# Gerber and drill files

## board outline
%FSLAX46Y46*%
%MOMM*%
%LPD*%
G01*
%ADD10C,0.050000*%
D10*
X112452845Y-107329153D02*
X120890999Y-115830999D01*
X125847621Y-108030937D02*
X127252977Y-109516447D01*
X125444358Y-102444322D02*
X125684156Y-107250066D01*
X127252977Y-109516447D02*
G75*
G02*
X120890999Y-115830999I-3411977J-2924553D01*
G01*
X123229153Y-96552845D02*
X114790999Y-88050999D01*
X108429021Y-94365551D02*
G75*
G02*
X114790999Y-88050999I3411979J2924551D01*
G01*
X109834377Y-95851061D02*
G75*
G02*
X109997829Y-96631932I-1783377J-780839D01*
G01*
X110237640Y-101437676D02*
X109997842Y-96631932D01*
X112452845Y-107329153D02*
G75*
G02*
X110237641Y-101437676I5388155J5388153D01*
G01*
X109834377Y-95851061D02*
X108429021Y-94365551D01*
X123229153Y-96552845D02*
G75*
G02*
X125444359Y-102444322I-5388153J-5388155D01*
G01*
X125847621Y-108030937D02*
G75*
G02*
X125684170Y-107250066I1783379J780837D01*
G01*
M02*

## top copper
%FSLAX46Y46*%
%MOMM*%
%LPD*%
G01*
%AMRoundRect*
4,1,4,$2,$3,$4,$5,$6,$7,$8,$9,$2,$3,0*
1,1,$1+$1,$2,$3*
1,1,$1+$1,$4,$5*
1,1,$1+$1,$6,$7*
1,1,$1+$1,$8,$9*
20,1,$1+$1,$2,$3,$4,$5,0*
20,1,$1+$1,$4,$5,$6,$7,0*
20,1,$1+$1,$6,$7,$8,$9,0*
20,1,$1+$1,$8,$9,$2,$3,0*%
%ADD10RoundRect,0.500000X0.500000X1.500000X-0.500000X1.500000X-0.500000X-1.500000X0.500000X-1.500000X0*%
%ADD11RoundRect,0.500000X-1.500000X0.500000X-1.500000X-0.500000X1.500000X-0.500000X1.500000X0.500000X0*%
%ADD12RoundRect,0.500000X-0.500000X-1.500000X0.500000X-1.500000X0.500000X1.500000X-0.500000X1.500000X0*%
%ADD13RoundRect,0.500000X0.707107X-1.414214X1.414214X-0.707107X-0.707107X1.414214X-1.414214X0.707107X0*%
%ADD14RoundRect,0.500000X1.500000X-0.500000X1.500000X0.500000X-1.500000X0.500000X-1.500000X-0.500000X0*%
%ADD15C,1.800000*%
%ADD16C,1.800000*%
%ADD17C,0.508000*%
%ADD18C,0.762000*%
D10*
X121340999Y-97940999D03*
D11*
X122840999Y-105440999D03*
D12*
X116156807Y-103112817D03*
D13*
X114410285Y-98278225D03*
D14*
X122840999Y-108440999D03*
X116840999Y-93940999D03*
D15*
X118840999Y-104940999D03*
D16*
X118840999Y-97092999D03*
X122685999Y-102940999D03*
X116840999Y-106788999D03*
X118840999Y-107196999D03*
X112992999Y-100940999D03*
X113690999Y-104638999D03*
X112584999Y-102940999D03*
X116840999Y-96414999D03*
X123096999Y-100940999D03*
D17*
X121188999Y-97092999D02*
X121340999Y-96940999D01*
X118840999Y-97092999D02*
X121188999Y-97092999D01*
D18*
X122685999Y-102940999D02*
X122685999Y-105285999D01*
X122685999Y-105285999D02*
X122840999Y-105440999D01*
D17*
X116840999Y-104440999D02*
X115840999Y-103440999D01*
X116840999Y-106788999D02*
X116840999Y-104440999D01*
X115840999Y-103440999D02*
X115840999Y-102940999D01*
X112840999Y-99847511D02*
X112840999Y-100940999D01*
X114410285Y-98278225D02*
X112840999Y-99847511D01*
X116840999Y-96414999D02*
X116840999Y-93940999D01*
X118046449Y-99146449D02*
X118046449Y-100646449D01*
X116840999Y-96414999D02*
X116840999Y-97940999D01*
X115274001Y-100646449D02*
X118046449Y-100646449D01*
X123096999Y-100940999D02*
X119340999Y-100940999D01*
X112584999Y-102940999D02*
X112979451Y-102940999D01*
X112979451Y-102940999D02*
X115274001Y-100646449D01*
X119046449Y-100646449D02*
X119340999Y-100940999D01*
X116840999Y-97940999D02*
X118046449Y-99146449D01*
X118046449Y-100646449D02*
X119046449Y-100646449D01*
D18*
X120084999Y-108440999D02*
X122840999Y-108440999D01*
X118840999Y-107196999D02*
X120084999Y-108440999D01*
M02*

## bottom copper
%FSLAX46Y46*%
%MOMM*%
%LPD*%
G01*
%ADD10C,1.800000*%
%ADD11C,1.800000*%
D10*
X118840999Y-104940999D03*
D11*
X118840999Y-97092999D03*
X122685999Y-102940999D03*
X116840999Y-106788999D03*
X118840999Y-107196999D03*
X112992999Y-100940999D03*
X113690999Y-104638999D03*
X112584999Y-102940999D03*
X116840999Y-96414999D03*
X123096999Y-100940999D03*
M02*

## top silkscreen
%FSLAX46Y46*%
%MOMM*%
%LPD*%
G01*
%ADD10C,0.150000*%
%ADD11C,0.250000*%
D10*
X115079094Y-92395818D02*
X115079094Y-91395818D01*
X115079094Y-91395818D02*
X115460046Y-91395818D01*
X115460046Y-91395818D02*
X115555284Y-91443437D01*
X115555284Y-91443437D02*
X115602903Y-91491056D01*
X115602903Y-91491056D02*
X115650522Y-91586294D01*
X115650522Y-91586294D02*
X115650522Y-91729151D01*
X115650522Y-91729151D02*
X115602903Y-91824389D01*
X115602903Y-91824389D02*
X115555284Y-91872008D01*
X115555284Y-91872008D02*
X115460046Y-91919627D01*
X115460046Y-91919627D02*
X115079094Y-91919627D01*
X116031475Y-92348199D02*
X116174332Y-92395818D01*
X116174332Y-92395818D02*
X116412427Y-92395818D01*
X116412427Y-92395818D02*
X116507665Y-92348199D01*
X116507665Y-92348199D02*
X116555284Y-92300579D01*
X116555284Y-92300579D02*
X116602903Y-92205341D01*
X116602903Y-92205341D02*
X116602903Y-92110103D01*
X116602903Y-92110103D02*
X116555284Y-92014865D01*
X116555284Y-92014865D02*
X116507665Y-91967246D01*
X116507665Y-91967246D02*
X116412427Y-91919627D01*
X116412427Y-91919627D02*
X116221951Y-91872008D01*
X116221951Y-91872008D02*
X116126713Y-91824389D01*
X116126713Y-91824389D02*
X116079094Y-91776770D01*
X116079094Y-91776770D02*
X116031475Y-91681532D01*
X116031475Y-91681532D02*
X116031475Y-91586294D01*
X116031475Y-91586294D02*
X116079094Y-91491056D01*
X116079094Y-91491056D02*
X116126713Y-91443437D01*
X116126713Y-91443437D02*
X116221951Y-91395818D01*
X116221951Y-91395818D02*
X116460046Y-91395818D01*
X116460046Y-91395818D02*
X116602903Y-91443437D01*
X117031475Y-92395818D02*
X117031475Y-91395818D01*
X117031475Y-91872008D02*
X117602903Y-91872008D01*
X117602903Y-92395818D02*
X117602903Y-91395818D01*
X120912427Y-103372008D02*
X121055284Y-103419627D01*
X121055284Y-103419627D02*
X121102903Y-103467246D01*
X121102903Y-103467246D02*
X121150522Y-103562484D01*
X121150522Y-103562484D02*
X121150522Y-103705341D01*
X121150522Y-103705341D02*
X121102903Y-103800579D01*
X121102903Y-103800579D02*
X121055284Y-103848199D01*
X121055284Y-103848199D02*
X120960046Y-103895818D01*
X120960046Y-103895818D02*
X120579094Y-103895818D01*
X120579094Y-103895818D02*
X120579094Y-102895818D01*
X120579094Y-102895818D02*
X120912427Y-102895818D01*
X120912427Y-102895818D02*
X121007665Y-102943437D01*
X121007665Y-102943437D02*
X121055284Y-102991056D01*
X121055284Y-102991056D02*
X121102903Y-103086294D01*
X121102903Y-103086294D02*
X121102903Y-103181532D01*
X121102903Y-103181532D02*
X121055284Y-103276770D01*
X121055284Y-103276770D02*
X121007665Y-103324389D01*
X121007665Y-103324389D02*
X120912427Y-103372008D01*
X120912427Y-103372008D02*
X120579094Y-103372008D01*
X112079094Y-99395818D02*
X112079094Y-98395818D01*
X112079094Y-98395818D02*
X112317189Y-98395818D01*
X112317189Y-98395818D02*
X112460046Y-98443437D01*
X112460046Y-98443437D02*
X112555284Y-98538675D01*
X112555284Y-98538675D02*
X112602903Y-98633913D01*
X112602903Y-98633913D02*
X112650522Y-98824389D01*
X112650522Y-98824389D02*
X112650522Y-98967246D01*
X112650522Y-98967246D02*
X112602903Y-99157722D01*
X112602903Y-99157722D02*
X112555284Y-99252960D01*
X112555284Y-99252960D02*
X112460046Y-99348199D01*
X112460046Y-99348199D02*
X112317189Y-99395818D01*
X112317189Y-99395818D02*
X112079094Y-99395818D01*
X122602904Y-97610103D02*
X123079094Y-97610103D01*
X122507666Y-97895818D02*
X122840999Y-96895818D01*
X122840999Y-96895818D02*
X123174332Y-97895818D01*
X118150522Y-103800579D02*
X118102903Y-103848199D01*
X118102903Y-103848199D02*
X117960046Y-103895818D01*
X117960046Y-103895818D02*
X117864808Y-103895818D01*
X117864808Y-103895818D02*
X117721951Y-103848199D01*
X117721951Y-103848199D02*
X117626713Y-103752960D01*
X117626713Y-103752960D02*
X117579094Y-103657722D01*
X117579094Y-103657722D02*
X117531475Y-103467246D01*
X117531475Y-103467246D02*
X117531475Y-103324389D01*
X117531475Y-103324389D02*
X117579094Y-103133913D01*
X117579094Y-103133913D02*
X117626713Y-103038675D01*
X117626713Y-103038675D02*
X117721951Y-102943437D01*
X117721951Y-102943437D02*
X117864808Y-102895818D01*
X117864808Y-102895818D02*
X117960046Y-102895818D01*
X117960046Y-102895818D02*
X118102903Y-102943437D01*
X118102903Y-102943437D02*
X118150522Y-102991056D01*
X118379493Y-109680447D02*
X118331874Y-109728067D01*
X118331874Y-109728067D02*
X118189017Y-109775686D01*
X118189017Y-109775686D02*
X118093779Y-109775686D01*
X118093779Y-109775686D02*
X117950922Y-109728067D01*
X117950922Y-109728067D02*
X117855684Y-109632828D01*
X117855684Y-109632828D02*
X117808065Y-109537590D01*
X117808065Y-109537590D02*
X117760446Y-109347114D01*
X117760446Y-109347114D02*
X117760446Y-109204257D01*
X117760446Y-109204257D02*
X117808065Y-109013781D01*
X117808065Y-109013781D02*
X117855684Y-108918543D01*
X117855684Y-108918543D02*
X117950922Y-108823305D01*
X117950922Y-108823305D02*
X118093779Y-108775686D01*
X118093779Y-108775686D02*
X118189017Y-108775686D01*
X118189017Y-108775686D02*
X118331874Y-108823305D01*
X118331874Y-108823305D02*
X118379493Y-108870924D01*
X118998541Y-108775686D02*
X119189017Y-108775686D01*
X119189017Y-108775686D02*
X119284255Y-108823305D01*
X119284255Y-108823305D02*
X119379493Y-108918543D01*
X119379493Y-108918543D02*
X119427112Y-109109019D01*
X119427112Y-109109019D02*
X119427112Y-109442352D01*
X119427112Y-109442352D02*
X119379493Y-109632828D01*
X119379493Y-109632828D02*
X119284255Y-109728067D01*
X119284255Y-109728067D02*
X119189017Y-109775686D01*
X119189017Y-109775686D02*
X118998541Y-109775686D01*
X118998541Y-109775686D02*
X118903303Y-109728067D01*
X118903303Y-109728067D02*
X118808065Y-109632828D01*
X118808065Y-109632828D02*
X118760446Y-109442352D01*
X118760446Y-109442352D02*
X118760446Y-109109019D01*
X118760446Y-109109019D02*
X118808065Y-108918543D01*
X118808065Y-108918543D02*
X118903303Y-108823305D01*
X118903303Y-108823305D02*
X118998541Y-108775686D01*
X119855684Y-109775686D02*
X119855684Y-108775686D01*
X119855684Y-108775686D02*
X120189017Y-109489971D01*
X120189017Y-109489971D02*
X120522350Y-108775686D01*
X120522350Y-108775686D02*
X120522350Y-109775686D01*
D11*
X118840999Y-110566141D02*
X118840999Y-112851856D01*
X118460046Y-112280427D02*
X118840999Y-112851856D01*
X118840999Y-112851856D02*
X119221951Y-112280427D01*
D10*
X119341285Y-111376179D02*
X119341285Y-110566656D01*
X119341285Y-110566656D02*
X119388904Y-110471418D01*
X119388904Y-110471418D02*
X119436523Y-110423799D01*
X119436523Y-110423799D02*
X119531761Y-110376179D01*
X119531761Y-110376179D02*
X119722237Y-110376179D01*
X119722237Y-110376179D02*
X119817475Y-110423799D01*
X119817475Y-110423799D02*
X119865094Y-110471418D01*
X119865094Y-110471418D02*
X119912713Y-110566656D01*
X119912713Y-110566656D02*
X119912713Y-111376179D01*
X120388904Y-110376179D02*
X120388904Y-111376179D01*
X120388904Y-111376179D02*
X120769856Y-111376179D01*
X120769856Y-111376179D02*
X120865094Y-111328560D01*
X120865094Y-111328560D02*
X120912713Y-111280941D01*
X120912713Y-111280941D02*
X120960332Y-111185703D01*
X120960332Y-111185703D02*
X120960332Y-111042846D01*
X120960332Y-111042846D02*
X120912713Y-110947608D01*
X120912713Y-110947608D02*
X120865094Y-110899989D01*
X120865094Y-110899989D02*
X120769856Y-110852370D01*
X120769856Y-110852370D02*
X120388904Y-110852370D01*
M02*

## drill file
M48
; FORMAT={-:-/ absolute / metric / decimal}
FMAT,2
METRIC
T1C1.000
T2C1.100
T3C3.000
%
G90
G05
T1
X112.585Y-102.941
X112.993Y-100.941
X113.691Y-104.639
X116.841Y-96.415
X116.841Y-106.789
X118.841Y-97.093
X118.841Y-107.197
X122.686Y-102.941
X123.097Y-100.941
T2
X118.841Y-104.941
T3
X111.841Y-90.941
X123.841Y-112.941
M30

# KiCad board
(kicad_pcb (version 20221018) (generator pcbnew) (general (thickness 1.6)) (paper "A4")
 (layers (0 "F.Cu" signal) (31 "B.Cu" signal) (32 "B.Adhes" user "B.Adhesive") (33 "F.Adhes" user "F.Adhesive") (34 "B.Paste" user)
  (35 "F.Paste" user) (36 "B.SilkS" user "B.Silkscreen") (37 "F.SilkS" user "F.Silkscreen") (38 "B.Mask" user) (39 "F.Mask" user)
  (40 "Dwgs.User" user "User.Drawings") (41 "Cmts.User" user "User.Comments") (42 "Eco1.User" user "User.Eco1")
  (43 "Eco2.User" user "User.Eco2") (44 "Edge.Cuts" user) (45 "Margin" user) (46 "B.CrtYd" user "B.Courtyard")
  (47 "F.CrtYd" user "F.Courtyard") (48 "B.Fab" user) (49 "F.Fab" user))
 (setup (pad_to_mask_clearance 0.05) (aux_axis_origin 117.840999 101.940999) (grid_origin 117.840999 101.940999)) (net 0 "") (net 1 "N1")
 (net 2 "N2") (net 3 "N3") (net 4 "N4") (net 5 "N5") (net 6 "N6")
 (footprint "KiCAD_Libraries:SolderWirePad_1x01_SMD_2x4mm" (layer "F.Cu") (at 121.340999 97.940999 180)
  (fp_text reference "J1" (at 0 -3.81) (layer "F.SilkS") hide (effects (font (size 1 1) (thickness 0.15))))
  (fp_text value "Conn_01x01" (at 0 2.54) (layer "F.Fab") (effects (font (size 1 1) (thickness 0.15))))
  (pad "1" smd roundrect (at 0 0 180) (size 2 4) (layers "F.Cu" "F.Paste" "F.Mask") (roundrect_rratio 0.25) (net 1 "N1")))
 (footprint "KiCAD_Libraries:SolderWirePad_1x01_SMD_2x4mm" (layer "F.Cu") (at 122.840999 105.440999 -90)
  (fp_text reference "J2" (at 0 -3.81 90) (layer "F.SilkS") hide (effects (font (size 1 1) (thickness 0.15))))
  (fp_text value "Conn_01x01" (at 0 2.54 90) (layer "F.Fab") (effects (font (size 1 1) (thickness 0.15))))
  (pad "1" smd roundrect (at 0 0 270) (size 2 4) (layers "F.Cu" "F.Paste" "F.Mask") (roundrect_rratio 0.25) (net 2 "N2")))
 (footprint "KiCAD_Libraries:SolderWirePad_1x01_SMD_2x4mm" (layer "F.Cu") (at 116.156807 103.112817)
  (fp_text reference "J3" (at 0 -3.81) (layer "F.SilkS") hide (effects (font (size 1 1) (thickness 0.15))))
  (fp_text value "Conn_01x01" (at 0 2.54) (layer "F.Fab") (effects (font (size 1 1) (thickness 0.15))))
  (pad "1" smd roundrect (at 0 0) (size 2 4) (layers "F.Cu" "F.Paste" "F.Mask") (roundrect_rratio 0.25) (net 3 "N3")))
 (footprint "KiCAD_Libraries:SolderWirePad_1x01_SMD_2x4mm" (layer "F.Cu") (at 114.410285 98.278225 45)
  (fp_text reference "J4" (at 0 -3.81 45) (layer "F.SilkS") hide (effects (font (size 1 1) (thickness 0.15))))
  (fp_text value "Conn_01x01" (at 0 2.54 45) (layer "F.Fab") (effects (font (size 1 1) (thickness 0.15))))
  (pad "1" smd roundrect (at 0 0 45) (size 2 4) (layers "F.Cu" "F.Paste" "F.Mask") (roundrect_rratio 0.25) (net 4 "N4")))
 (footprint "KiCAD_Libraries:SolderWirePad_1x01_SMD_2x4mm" (layer "F.Cu") (at 122.840999 108.440999 90)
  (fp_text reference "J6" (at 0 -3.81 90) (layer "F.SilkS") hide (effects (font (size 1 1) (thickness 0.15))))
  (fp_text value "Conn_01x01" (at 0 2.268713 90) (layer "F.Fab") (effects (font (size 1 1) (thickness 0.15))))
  (pad "1" smd roundrect (at 0 0 90) (size 2 4) (layers "F.Cu" "F.Paste" "F.Mask") (roundrect_rratio 0.25) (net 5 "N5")))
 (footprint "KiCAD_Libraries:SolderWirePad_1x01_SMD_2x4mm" (layer "F.Cu") (at 116.840999 93.940999 90)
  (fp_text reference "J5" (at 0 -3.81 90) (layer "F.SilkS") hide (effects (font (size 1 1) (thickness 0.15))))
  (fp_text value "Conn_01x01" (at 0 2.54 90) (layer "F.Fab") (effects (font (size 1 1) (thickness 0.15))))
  (pad "1" smd roundrect (at 0 0 90) (size 2 4) (layers "F.Cu" "F.Paste" "F.Mask") (roundrect_rratio 0.25) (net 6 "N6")))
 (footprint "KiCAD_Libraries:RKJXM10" (layer "B.Cu") (at 117.840999 101.940999)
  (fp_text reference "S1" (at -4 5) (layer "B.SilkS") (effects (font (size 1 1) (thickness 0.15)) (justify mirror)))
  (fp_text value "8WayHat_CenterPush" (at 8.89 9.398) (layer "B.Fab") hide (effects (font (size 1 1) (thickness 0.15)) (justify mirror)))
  (pad "" np_thru_hole circle (at 1 3) (size 1.8 1.8) (drill 1.1) (layers "*.Cu" "*.Mask"))
  (pad "A" thru_hole circle (at 1 -4.848) (size 1.8 1.8) (drill 1) (layers "*.Cu" "*.Mask") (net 1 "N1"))
  (pad "B" thru_hole circle (at 4.845 1) (size 1.8 1.8) (drill 1) (layers "*.Cu" "*.Mask") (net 2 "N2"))
  (pad "C" thru_hole circle (at -1 4.848) (size 1.8 1.8) (drill 1) (layers "*.Cu" "*.Mask") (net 3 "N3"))
  (pad "COM" thru_hole circle (at 1 5.256) (size 1.8 1.8) (drill 1) (layers "*.Cu" "*.Mask") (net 5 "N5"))
  (pad "D" thru_hole circle (at -4.848 -1) (size 1.8 1.8) (drill 1) (layers "*.Cu" "*.Mask") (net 4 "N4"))
  (pad "GND" thru_hole circle (at -4.15 2.698) (size 1.8 1.8) (drill 1) (layers "*.Cu" "*.Mask"))
  (pad "PUSH1" thru_hole circle (at -5.256 1) (size 1.8 1.8) (drill 1) (layers "*.Cu" "*.Mask") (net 6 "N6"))
  (pad "PUSH2" thru_hole circle (at -1 -5.526) (size 1.8 1.8) (drill 1) (layers "*.Cu" "*.Mask") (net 6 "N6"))
  (pad "PUSH3" thru_hole circle (at 5.256 -1) (size 1.8 1.8) (drill 1) (layers "*.Cu" "*.Mask") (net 6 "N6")))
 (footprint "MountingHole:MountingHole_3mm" (layer "B.Cu") (at 123.840999 112.940999)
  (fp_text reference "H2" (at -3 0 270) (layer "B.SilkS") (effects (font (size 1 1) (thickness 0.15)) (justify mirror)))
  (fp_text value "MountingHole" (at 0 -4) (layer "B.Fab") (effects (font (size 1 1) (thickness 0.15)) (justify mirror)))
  (pad "" np_thru_hole circle (at 0 0) (size 3 3) (drill 3) (layers "*.Cu" "*.Mask")))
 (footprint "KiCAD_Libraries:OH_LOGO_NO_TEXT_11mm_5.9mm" (layer "B.Cu") (at 118.340999 101.440999 -160)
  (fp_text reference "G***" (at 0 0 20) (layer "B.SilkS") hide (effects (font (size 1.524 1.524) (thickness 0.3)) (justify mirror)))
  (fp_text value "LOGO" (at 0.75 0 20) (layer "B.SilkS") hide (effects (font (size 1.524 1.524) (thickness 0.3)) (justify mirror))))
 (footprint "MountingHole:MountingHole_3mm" (layer "B.Cu") (at 111.840999 90.940999 180)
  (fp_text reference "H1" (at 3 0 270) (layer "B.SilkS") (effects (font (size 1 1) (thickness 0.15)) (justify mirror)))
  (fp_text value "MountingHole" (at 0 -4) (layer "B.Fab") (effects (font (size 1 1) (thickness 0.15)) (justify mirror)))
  (pad "" np_thru_hole circle (at 0 0 180) (size 3 3) (drill 3) (layers "*.Cu" "*.Mask")))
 (gr_line (start 112.452845 107.329153) (end 120.890999 115.830999) (stroke (width 0.05) (type solid)) (layer "Edge.Cuts"))
 (gr_line (start 125.847621 108.030937) (end 127.252977 109.516447) (stroke (width 0.05) (type solid)) (layer "Edge.Cuts"))
 (gr_line (start 125.444358 102.444322) (end 125.684156 107.250066) (stroke (width 0.05) (type solid)) (layer "Edge.Cuts"))
 (gr_arc (start 127.252977 109.516447) (mid 127.006713 115.63049) (end 120.890999 115.830999) (stroke (width 0.05) (type solid))
  (layer "Edge.Cuts"))
 (gr_line (start 123.229153 96.552845) (end 114.790999 88.050999) (stroke (width 0.05) (type solid)) (layer "Edge.Cuts"))
 (gr_arc (start 108.429021 94.365551) (mid 108.675285 88.251508) (end 114.790999 88.050999) (stroke (width 0.05) (type solid))
  (layer "Edge.Cuts"))
 (gr_arc (start 109.834377 95.851061) (mid 109.956537 96.233033) (end 109.997842 96.631932) (stroke (width 0.05) (type solid))
  (layer "Edge.Cuts"))
 (gr_line (start 110.23764 101.437676) (end 109.997842 96.631932) (stroke (width 0.05) (type solid)) (layer "Edge.Cuts"))
 (gr_arc (start 112.452845 107.329153) (mid 110.708522 104.622822) (end 110.23764 101.437676) (stroke (width 0.05) (type solid))
  (layer "Edge.Cuts"))
 (gr_line (start 109.834377 95.851061) (end 108.429021 94.365551) (stroke (width 0.05) (type solid)) (layer "Edge.Cuts"))
 (gr_arc (start 123.229153 96.552845) (mid 124.973476 99.259176) (end 125.444358 102.444322) (stroke (width 0.05) (type solid))
  (layer "Edge.Cuts"))
 (gr_arc (start 125.847621 108.030937) (mid 125.725461 107.648965) (end 125.684156 107.250066) (stroke (width 0.05) (type solid))
  (layer "Edge.Cuts"))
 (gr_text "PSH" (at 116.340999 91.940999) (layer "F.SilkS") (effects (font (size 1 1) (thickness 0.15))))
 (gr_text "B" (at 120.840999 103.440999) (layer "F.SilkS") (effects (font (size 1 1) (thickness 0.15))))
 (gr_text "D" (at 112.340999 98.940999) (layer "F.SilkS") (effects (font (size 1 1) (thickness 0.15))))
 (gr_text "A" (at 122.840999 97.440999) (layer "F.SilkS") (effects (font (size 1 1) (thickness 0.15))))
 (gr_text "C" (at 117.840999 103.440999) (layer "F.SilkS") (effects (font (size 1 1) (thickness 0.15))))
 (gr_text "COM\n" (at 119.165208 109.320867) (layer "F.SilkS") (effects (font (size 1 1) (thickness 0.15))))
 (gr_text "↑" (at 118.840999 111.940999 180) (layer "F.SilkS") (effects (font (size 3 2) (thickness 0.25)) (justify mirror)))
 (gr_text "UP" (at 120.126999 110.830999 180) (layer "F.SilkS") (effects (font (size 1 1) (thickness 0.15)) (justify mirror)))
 (segment (start 121.188999 97.092999) (end 121.340999 96.940999) (width 0.508) (layer "F.Cu") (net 1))
 (segment (start 118.840999 97.092999) (end 121.188999 97.092999) (width 0.508) (layer "F.Cu") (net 1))
 (segment (start 122.685999 102.940999) (end 122.685999 105.285999) (width 0.762) (layer "F.Cu") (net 2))
 (segment (start 122.685999 105.285999) (end 122.840999 105.440999) (width 0.762) (layer "F.Cu") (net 2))
 (segment (start 116.840999 104.440999) (end 115.840999 103.440999) (width 0.508) (layer "F.Cu") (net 3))
 (segment (start 116.840999 106.788999) (end 116.840999 104.440999) (width 0.508) (layer "F.Cu") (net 3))
 (segment (start 115.840999 103.440999) (end 115.840999 102.940999) (width 0.508) (layer "F.Cu") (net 3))
 (segment (start 112.840999 99.847511) (end 112.840999 100.940999) (width 0.508) (layer "F.Cu") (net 4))
 (segment (start 114.410285 98.278225) (end 112.840999 99.847511) (width 0.508) (layer "F.Cu") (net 4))
 (segment (start 116.840999 96.414999) (end 116.840999 93.940999) (width 0.508) (layer "F.Cu") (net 6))
 (segment (start 118.046449 99.146449) (end 118.046449 100.646449) (width 0.508) (layer "F.Cu") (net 6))
 (segment (start 116.840999 96.414999) (end 116.840999 97.940999) (width 0.508) (layer "F.Cu") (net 6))
 (segment (start 115.274001 100.646449) (end 118.046449 100.646449) (width 0.508) (layer "F.Cu") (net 6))
 (segment (start 123.096999 100.940999) (end 119.340999 100.940999) (width 0.508) (layer "F.Cu") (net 6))
 (segment (start 112.584999 102.940999) (end 112.979451 102.940999) (width 0.508) (layer "F.Cu") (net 6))
 (segment (start 112.979451 102.940999) (end 115.274001 100.646449) (width 0.508) (layer "F.Cu") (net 6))
 (segment (start 119.046449 100.646449) (end 119.340999 100.940999) (width 0.508) (layer "F.Cu") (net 6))
 (segment (start 116.840999 97.940999) (end 118.046449 99.146449) (width 0.508) (layer "F.Cu") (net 6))
 (segment (start 118.046449 100.646449) (end 119.046449 100.646449) (width 0.508) (layer "F.Cu") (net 6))
 (segment (start 120.084999 108.440999) (end 122.840999 108.440999) (width 0.762) (layer "F.Cu") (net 5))
 (segment (start 118.840999 107.196999) (end 120.084999 108.440999) (width 0.762) (layer "F.Cu") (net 5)))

